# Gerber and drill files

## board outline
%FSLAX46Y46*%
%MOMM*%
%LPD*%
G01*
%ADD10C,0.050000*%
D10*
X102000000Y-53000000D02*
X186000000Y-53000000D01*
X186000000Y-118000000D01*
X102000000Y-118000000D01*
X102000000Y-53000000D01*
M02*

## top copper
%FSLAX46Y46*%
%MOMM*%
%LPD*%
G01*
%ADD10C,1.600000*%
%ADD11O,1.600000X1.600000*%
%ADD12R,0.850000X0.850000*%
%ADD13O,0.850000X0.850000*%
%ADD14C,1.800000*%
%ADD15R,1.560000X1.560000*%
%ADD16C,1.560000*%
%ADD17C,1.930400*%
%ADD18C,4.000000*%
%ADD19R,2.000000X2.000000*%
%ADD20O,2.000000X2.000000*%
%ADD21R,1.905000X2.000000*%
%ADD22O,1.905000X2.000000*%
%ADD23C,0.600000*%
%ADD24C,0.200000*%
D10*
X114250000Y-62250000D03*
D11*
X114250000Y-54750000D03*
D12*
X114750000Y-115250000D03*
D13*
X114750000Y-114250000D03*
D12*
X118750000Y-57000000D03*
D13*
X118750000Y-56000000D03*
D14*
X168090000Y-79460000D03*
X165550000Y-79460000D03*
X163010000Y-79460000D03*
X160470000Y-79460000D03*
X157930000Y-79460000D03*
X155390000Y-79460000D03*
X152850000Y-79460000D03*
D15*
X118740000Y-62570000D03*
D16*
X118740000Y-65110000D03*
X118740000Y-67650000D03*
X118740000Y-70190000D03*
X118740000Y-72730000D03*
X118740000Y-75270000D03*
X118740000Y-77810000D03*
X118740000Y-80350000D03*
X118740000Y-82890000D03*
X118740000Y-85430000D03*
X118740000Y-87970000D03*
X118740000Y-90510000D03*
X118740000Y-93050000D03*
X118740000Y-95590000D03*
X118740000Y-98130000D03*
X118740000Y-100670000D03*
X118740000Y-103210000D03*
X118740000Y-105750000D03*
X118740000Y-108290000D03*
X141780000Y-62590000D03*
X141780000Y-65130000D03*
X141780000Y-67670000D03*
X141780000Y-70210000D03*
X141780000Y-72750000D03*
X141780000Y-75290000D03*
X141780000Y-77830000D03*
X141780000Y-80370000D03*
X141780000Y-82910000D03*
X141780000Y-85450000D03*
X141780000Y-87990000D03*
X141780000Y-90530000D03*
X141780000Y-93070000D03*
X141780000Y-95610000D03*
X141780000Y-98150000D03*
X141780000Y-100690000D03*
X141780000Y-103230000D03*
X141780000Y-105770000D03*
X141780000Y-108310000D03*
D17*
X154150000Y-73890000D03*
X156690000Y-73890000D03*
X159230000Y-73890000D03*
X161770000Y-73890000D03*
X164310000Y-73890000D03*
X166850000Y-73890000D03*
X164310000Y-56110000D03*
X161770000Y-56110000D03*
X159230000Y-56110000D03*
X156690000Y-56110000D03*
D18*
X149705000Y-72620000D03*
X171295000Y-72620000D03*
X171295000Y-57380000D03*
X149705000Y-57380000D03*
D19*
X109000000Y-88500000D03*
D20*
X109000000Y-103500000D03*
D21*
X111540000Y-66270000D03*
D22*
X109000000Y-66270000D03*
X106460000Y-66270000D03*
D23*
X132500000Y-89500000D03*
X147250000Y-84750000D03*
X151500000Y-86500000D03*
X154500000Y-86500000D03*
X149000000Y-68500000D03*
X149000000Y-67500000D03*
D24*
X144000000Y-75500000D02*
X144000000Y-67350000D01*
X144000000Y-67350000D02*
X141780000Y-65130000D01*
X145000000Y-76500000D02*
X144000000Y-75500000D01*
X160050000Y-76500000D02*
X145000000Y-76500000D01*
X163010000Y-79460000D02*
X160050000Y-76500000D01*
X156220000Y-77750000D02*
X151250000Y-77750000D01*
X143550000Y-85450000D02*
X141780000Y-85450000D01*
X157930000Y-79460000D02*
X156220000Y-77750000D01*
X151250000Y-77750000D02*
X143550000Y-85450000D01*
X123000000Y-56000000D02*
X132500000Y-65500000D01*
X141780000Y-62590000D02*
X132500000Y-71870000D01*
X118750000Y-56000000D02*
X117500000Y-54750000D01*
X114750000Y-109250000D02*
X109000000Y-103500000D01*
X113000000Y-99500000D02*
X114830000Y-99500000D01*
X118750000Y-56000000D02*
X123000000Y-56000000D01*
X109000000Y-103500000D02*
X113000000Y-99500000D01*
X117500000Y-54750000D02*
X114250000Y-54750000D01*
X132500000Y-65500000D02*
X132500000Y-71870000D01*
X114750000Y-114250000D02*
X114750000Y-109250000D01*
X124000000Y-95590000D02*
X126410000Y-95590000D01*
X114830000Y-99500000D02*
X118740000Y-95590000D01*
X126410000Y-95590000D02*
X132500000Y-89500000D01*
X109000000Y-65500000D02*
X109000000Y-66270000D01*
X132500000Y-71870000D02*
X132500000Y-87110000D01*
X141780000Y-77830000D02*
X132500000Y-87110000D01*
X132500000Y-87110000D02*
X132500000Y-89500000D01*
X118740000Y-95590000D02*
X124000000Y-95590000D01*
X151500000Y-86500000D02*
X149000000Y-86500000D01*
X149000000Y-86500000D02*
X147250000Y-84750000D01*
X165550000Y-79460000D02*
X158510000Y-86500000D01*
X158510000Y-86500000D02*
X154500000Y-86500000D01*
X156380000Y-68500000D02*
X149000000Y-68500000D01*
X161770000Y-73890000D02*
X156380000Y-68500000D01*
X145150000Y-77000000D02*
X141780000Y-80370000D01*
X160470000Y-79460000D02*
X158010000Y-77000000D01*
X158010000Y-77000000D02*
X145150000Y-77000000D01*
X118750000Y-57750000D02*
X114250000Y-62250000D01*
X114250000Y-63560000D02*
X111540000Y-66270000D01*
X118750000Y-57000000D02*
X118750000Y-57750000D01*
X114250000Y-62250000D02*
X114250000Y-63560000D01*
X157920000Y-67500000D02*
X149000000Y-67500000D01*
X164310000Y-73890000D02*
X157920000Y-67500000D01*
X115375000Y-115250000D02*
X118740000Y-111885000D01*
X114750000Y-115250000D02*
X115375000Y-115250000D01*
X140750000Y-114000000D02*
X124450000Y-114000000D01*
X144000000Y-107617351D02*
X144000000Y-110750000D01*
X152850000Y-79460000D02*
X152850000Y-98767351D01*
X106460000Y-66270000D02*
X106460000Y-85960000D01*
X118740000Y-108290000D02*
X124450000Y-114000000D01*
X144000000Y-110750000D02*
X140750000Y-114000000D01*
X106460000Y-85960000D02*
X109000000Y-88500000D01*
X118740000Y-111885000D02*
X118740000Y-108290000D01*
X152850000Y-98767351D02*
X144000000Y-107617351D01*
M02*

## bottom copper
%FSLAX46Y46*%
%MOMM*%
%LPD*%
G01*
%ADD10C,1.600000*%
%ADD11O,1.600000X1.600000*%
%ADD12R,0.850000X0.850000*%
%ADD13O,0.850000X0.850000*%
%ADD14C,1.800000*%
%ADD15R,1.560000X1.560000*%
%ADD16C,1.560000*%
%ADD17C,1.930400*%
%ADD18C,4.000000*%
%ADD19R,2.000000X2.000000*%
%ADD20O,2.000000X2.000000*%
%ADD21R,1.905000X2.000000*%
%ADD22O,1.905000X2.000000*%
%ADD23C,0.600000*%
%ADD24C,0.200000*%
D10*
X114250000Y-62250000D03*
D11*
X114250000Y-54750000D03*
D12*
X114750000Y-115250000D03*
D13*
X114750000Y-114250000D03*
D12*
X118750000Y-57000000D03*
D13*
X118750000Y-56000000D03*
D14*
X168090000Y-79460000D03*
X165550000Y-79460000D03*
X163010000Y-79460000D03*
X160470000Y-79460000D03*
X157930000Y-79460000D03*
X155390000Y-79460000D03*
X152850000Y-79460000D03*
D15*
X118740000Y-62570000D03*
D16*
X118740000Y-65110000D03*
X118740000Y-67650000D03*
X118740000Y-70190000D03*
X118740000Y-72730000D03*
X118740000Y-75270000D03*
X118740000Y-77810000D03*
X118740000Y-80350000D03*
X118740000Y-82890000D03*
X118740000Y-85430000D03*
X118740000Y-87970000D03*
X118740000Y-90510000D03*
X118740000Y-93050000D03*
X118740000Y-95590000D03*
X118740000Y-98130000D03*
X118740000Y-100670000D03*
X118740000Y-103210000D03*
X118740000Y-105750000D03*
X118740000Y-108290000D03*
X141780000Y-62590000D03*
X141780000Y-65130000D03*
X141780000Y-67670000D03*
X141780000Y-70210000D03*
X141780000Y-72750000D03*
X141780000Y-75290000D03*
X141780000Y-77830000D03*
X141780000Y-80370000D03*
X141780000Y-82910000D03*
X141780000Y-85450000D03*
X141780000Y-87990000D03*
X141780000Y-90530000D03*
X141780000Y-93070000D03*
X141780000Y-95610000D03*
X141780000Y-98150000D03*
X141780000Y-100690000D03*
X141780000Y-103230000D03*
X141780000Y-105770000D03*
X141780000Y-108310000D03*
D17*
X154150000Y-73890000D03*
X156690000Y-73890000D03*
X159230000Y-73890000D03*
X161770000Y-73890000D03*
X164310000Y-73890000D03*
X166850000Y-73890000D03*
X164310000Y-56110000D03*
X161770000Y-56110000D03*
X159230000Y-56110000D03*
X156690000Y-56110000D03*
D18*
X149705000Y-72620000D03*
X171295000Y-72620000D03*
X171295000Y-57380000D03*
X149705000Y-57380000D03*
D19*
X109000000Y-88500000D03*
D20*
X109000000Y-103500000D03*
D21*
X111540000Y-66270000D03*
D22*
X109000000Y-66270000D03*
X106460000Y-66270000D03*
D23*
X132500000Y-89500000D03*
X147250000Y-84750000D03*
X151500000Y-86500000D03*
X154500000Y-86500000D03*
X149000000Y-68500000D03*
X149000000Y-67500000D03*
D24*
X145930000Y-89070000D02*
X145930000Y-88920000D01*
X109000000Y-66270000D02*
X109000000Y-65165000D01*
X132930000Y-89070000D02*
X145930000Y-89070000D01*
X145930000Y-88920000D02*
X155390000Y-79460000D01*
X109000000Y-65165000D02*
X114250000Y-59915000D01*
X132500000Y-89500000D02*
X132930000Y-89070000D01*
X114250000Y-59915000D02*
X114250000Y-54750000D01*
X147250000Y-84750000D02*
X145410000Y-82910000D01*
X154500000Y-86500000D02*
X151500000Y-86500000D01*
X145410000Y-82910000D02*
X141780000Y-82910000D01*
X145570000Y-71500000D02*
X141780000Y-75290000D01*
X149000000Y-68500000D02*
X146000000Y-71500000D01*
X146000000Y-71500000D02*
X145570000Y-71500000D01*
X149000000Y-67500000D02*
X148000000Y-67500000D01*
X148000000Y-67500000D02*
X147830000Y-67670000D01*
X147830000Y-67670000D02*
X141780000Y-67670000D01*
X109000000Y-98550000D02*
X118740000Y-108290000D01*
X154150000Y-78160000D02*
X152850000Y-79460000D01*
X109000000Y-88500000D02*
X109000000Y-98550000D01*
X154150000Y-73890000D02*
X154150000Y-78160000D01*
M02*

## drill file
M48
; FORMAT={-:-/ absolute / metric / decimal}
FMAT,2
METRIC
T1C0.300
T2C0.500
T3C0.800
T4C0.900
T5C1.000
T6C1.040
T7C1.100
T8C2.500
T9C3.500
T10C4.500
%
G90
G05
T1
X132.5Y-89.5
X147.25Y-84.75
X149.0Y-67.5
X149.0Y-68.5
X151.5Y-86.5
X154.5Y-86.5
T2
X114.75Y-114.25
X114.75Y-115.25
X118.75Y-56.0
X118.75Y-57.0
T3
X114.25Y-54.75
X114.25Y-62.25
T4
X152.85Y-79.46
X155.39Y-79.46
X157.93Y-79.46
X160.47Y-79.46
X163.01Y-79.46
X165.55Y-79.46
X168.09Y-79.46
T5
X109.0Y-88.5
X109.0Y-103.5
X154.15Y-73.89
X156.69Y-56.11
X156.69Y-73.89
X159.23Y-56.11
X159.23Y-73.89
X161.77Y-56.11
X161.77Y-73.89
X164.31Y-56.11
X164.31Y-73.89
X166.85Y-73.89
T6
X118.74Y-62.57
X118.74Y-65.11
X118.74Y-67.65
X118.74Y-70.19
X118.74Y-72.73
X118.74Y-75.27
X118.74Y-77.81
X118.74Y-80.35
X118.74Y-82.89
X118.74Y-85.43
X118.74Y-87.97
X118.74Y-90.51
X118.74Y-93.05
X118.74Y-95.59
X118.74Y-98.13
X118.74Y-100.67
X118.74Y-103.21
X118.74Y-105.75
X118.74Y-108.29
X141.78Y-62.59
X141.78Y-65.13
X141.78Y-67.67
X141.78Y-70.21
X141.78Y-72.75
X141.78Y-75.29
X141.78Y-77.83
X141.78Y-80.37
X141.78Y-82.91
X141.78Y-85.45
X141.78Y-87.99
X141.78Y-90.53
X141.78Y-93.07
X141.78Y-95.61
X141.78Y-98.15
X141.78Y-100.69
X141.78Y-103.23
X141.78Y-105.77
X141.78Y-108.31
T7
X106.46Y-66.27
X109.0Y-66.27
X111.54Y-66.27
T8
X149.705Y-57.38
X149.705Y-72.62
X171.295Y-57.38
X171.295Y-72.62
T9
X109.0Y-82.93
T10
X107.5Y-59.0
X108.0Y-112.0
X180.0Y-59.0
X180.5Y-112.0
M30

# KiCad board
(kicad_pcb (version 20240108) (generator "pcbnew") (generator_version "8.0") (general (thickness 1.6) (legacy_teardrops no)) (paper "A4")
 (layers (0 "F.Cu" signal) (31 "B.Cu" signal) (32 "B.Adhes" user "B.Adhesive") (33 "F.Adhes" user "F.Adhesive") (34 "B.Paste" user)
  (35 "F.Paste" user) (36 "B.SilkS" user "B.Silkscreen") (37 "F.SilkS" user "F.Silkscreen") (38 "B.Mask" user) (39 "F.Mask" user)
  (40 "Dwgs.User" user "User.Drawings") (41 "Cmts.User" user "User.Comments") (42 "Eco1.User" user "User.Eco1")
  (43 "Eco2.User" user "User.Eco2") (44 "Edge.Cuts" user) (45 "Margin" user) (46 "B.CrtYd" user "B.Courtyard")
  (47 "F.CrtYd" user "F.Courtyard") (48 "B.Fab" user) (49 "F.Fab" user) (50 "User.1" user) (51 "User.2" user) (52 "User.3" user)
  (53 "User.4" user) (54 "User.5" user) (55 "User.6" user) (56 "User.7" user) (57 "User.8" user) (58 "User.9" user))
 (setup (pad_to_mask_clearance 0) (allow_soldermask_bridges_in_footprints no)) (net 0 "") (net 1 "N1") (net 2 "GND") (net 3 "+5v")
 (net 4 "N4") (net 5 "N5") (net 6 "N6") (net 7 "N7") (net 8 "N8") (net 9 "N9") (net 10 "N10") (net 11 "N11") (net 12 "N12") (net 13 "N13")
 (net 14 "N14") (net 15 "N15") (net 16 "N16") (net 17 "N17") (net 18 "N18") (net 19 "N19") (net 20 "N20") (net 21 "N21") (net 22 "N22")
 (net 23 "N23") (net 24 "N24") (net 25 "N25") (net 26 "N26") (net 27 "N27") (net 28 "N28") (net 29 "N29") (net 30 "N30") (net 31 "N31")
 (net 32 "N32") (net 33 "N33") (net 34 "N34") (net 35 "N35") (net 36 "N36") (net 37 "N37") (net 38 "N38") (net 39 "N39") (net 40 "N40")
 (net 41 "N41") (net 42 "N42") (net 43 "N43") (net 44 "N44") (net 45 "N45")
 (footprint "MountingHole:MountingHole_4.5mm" (layer "F.Cu") (at 107.5 59)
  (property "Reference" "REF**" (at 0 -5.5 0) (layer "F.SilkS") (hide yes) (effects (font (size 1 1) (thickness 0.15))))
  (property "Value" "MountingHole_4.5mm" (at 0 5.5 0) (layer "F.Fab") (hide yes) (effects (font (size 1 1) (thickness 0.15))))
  (pad "" np_thru_hole circle (at 0 0) (size 4.5 4.5) (drill 4.5) (layers "*.Cu" "*.Mask")))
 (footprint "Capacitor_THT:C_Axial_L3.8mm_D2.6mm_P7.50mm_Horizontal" (layer "F.Cu") (at 114.25 62.25 90)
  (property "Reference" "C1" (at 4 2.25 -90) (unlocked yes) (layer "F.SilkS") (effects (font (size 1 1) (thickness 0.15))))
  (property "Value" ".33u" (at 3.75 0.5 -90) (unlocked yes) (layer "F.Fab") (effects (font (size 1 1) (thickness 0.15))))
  (pad "1" thru_hole circle (at 0 0 90) (size 1.6 1.6) (drill 0.8) (layers "*.Cu" "*.Mask") (remove_unused_layers no) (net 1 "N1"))
  (pad "2" thru_hole oval (at 7.5 0 90) (size 1.6 1.6) (drill 0.8) (layers "*.Cu" "*.Mask") (remove_unused_layers no) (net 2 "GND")))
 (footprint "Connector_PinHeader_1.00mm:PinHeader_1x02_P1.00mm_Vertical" (layer "F.Cu") (at 114.75 115.25 180)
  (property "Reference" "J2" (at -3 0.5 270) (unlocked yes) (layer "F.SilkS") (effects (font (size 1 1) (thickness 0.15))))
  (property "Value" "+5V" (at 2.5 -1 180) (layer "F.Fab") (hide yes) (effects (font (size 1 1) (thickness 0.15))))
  (pad "1" thru_hole rect (at 0 0 180) (size 0.85 0.85) (drill 0.5) (layers "*.Cu" "*.Mask") (remove_unused_layers no) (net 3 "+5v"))
  (pad "2" thru_hole oval (at 0 1 180) (size 0.85 0.85) (drill 0.5) (layers "*.Cu" "*.Mask") (remove_unused_layers no) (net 2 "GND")))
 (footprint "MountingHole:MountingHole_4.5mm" (layer "F.Cu") (at 180.5 112)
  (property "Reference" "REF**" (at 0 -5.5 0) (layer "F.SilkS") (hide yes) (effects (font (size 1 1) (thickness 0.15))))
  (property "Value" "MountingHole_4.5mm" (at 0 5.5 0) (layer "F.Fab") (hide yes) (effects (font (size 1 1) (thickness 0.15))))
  (pad "" np_thru_hole circle (at 0 0) (size 4.5 4.5) (drill 4.5) (layers "*.Cu" "*.Mask")))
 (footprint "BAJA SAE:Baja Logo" (layer "F.Cu") (at 181.25 79.5 -90)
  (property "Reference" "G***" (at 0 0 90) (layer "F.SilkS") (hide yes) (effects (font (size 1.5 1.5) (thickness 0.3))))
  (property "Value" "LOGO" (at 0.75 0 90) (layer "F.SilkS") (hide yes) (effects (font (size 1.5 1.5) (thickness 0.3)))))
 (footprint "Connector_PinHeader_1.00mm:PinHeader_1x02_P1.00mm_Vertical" (layer "F.Cu") (at 118.75 57 180)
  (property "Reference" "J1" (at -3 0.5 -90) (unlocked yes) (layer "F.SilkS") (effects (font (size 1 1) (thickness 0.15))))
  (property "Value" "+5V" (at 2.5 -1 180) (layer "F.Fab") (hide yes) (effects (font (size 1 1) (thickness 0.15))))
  (pad "1" thru_hole rect (at 0 0 180) (size 0.85 0.85) (drill 0.5) (layers "*.Cu" "*.Mask") (remove_unused_layers no) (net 1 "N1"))
  (pad "2" thru_hole oval (at 0 1 180) (size 0.85 0.85) (drill 0.5) (layers "*.Cu" "*.Mask") (remove_unused_layers no) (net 2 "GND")))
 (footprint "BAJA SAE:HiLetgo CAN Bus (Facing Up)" (layer "F.Cu") (at 160.5 97.5 -90)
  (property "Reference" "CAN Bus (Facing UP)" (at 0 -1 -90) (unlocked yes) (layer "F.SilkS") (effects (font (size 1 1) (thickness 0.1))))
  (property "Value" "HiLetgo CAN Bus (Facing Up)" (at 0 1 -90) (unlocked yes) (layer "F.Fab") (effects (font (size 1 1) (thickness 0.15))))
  (pad "1" thru_hole circle (at -18.04 -7.59 270) (size 1.8 1.8) (drill 0.9) (layers "*.Cu" "*.Mask") (remove_unused_layers no) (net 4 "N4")
   (solder_mask_margin 0.102))
  (pad "2" thru_hole circle (at -18.04 -5.05 270) (size 1.8 1.8) (drill 0.9) (layers "*.Cu" "*.Mask") (remove_unused_layers no) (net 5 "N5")
   (solder_mask_margin 0.102))
  (pad "3" thru_hole circle (at -18.04 -2.51 270) (size 1.8 1.8) (drill 0.9) (layers "*.Cu" "*.Mask") (remove_unused_layers no) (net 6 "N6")
   (solder_mask_margin 0.102))
  (pad "4" thru_hole circle (at -18.04 0.03 270) (size 1.8 1.8) (drill 0.9) (layers "*.Cu" "*.Mask") (remove_unused_layers no) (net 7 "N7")
   (solder_mask_margin 0.102))
  (pad "5" thru_hole circle (at -18.04 2.57 270) (size 1.8 1.8) (drill 0.9) (layers "*.Cu" "*.Mask") (remove_unused_layers no) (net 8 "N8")
   (solder_mask_margin 0.102))
  (pad "6" thru_hole circle (at -18.04 5.11 270) (size 1.8 1.8) (drill 0.9) (layers "*.Cu" "*.Mask") (remove_unused_layers no) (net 2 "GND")
   (solder_mask_margin 0.102))
  (pad "7" thru_hole circle (at -18.04 7.65 270) (size 1.8 1.8) (drill 0.9) (layers "*.Cu" "*.Mask") (remove_unused_layers no) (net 3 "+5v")
   (solder_mask_margin 0.102)))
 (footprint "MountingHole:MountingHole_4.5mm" (layer "F.Cu") (at 180 59)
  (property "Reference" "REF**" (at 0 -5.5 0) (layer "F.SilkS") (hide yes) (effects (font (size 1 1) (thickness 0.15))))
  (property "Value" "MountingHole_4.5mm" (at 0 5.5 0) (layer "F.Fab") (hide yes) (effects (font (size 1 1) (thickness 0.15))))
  (pad "" np_thru_hole circle (at 0 0) (size 4.5 4.5) (drill 4.5) (layers "*.Cu" "*.Mask")))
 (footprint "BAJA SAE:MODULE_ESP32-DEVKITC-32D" (layer "F.Cu") (at 130.5 81.5)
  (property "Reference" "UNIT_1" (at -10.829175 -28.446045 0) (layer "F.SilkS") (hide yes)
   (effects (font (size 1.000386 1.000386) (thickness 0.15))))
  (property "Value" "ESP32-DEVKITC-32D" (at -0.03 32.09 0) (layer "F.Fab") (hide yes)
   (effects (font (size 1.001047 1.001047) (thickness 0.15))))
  (pad "J2-1" thru_hole rect (at -11.76 -18.93) (size 1.56 1.56) (drill 1.04) (layers "*.Cu" "*.Mask") (remove_unused_layers no)
   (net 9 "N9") (solder_mask_margin 0.102))
  (pad "J2-2" thru_hole circle (at -11.76 -16.39) (size 1.56 1.56) (drill 1.04) (layers "*.Cu" "*.Mask") (remove_unused_layers no)
   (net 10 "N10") (solder_mask_margin 0.102))
  (pad "J2-3" thru_hole circle (at -11.76 -13.85) (size 1.56 1.56) (drill 1.04) (layers "*.Cu" "*.Mask") (remove_unused_layers no)
   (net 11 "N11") (solder_mask_margin 0.102))
  (pad "J2-4" thru_hole circle (at -11.76 -11.31) (size 1.56 1.56) (drill 1.04) (layers "*.Cu" "*.Mask") (remove_unused_layers no)
   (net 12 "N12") (solder_mask_margin 0.102))
  (pad "J2-5" thru_hole circle (at -11.76 -8.77) (size 1.56 1.56) (drill 1.04) (layers "*.Cu" "*.Mask") (remove_unused_layers no)
   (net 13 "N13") (solder_mask_margin 0.102))
  (pad "J2-6" thru_hole circle (at -11.76 -6.23) (size 1.56 1.56) (drill 1.04) (layers "*.Cu" "*.Mask") (remove_unused_layers no)
   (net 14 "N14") (solder_mask_margin 0.102))
  (pad "J2-7" thru_hole circle (at -11.76 -3.69) (size 1.56 1.56) (drill 1.04) (layers "*.Cu" "*.Mask") (remove_unused_layers no)
   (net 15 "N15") (solder_mask_margin 0.102))
  (pad "J2-8" thru_hole circle (at -11.76 -1.15) (size 1.56 1.56) (drill 1.04) (layers "*.Cu" "*.Mask") (remove_unused_layers no)
   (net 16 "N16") (solder_mask_margin 0.102))
  (pad "J2-9" thru_hole circle (at -11.76 1.39) (size 1.56 1.56) (drill 1.04) (layers "*.Cu" "*.Mask") (remove_unused_layers no)
   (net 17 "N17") (solder_mask_margin 0.102))
  (pad "J2-10" thru_hole circle (at -11.76 3.93) (size 1.56 1.56) (drill 1.04) (layers "*.Cu" "*.Mask") (remove_unused_layers no)
   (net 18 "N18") (solder_mask_margin 0.102))
  (pad "J2-11" thru_hole circle (at -11.76 6.47) (size 1.56 1.56) (drill 1.04) (layers "*.Cu" "*.Mask") (remove_unused_layers no)
   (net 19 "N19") (solder_mask_margin 0.102))
  (pad "J2-12" thru_hole circle (at -11.76 9.01) (size 1.56 1.56) (drill 1.04) (layers "*.Cu" "*.Mask") (remove_unused_layers no)
   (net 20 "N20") (solder_mask_margin 0.102))
  (pad "J2-13" thru_hole circle (at -11.76 11.55) (size 1.56 1.56) (drill 1.04) (layers "*.Cu" "*.Mask") (remove_unused_layers no)
   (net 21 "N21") (solder_mask_margin 0.102))
  (pad "J2-14" thru_hole circle (at -11.76 14.09) (size 1.56 1.56) (drill 1.04) (layers "*.Cu" "*.Mask") (remove_unused_layers no)
   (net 2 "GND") (solder_mask_margin 0.102))
  (pad "J2-15" thru_hole circle (at -11.76 16.63) (size 1.56 1.56) (drill 1.04) (layers "*.Cu" "*.Mask") (remove_unused_layers no)
   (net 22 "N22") (solder_mask_margin 0.102))
  (pad "J2-16" thru_hole circle (at -11.76 19.17) (size 1.56 1.56) (drill 1.04) (layers "*.Cu" "*.Mask") (remove_unused_layers no)
   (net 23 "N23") (solder_mask_margin 0.102))
  (pad "J2-17" thru_hole circle (at -11.76 21.71) (size 1.56 1.56) (drill 1.04) (layers "*.Cu" "*.Mask") (remove_unused_layers no)
   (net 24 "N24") (solder_mask_margin 0.102))
  (pad "J2-18" thru_hole circle (at -11.76 24.25) (size 1.56 1.56) (drill 1.04) (layers "*.Cu" "*.Mask") (remove_unused_layers no)
   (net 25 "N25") (solder_mask_margin 0.102))
  (pad "J2-19" thru_hole circle (at -11.76 26.79) (size 1.56 1.56) (drill 1.04) (layers "*.Cu" "*.Mask") (remove_unused_layers no)
   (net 3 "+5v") (solder_mask_margin 0.102))
  (pad "J3-1" thru_hole circle (at 11.28 -18.91) (size 1.56 1.56) (drill 1.04) (layers "*.Cu" "*.Mask") (remove_unused_layers no)
   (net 2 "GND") (solder_mask_margin 0.102))
  (pad "J3-2" thru_hole circle (at 11.28 -16.37) (size 1.56 1.56) (drill 1.04) (layers "*.Cu" "*.Mask") (remove_unused_layers no)
   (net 6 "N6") (solder_mask_margin 0.102))
  (pad "J3-3" thru_hole circle (at 11.28 -13.83) (size 1.56 1.56) (drill 1.04) (layers "*.Cu" "*.Mask") (remove_unused_layers no)
   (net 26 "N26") (solder_mask_margin 0.102))
  (pad "J3-4" thru_hole circle (at 11.28 -11.29) (size 1.56 1.56) (drill 1.04) (layers "*.Cu" "*.Mask") (remove_unused_layers no)
   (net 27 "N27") (solder_mask_margin 0.102))
  (pad "J3-5" thru_hole circle (at 11.28 -8.75) (size 1.56 1.56) (drill 1.04) (layers "*.Cu" "*.Mask") (remove_unused_layers no)
   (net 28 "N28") (solder_mask_margin 0.102))
  (pad "J3-6" thru_hole circle (at 11.28 -6.21) (size 1.56 1.56) (drill 1.04) (layers "*.Cu" "*.Mask") (remove_unused_layers no)
   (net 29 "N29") (solder_mask_margin 0.102))
  (pad "J3-7" thru_hole circle (at 11.28 -3.67) (size 1.56 1.56) (drill 1.04) (layers "*.Cu" "*.Mask") (remove_unused_layers no)
   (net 2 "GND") (solder_mask_margin 0.102))
  (pad "J3-8" thru_hole circle (at 11.28 -1.13) (size 1.56 1.56) (drill 1.04) (layers "*.Cu" "*.Mask") (remove_unused_layers no)
   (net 7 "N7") (solder_mask_margin 0.102))
  (pad "J3-9" thru_hole circle (at 11.28 1.41) (size 1.56 1.56) (drill 1.04) (layers "*.Cu" "*.Mask") (remove_unused_layers no) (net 5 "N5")
   (solder_mask_margin 0.102))
  (pad "J3-10" thru_hole circle (at 11.28 3.95) (size 1.56 1.56) (drill 1.04) (layers "*.Cu" "*.Mask") (remove_unused_layers no)
   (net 8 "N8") (solder_mask_margin 0.102))
  (pad "J3-11" thru_hole circle (at 11.28 6.49) (size 1.56 1.56) (drill 1.04) (layers "*.Cu" "*.Mask") (remove_unused_layers no)
   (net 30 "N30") (solder_mask_margin 0.102))
  (pad "J3-12" thru_hole circle (at 11.28 9.03) (size 1.56 1.56) (drill 1.04) (layers "*.Cu" "*.Mask") (remove_unused_layers no)
   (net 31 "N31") (solder_mask_margin 0.102))
  (pad "J3-13" thru_hole circle (at 11.28 11.57) (size 1.56 1.56) (drill 1.04) (layers "*.Cu" "*.Mask") (remove_unused_layers no)
   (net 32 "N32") (solder_mask_margin 0.102))
  (pad "J3-14" thru_hole circle (at 11.28 14.11) (size 1.56 1.56) (drill 1.04) (layers "*.Cu" "*.Mask") (remove_unused_layers no)
   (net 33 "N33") (solder_mask_margin 0.102))
  (pad "J3-15" thru_hole circle (at 11.28 16.65) (size 1.56 1.56) (drill 1.04) (layers "*.Cu" "*.Mask") (remove_unused_layers no)
   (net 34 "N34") (solder_mask_margin 0.102))
  (pad "J3-16" thru_hole circle (at 11.28 19.19) (size 1.56 1.56) (drill 1.04) (layers "*.Cu" "*.Mask") (remove_unused_layers no)
   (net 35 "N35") (solder_mask_margin 0.102))
  (pad "J3-17" thru_hole circle (at 11.28 21.73) (size 1.56 1.56) (drill 1.04) (layers "*.Cu" "*.Mask") (remove_unused_layers no)
   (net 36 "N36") (solder_mask_margin 0.102))
  (pad "J3-18" thru_hole circle (at 11.28 24.27) (size 1.56 1.56) (drill 1.04) (layers "*.Cu" "*.Mask") (remove_unused_layers no)
   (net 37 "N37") (solder_mask_margin 0.102))
  (pad "J3-19" thru_hole circle (at 11.28 26.81) (size 1.56 1.56) (drill 1.04) (layers "*.Cu" "*.Mask") (remove_unused_layers no)
   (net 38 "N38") (solder_mask_margin 0.102)))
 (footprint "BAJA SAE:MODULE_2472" (layer "F.Cu") (at 160.5 65)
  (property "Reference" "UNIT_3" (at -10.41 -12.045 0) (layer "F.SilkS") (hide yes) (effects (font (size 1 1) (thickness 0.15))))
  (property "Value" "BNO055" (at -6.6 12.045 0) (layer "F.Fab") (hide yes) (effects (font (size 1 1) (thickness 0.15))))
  (pad "1" thru_hole circle (at -6.35 8.89) (size 1.9304 1.9304) (drill 1) (layers "*.Cu" "*.Mask") (remove_unused_layers no) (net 3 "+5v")
   (solder_mask_margin 0.102))
  (pad "2" thru_hole circle (at -3.81 8.89) (size 1.9304 1.9304) (drill 1) (layers "*.Cu" "*.Mask") (remove_unused_layers no) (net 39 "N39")
   (solder_mask_margin 0.102))
  (pad "3" thru_hole circle (at -1.27 8.89) (size 1.9304 1.9304) (drill 1) (layers "*.Cu" "*.Mask") (remove_unused_layers no) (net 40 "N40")
   (solder_mask_margin 0.102))
  (pad "4" thru_hole circle (at 1.27 8.89) (size 1.9304 1.9304) (drill 1) (layers "*.Cu" "*.Mask") (remove_unused_layers no) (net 29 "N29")
   (solder_mask_margin 0.102))
  (pad "5" thru_hole circle (at 3.81 8.89) (size 1.9304 1.9304) (drill 1) (layers "*.Cu" "*.Mask") (remove_unused_layers no) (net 26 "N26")
   (solder_mask_margin 0.102))
  (pad "6" thru_hole circle (at 6.35 8.89) (size 1.9304 1.9304) (drill 1) (layers "*.Cu" "*.Mask") (remove_unused_layers no) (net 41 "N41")
   (solder_mask_margin 0.102))
  (pad "7" thru_hole circle (at 3.81 -8.89) (size 1.9304 1.9304) (drill 1) (layers "*.Cu" "*.Mask") (remove_unused_layers no) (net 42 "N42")
   (solder_mask_margin 0.102))
  (pad "8" thru_hole circle (at 1.27 -8.89) (size 1.9304 1.9304) (drill 1) (layers "*.Cu" "*.Mask") (remove_unused_layers no) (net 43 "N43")
   (solder_mask_margin 0.102))
  (pad "9" thru_hole circle (at -1.27 -8.89) (size 1.9304 1.9304) (drill 1) (layers "*.Cu" "*.Mask") (remove_unused_layers no)
   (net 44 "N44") (solder_mask_margin 0.102))
  (pad "10" thru_hole circle (at -3.81 -8.89) (size 1.9304 1.9304) (drill 1) (layers "*.Cu" "*.Mask") (remove_unused_layers no)
   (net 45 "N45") (solder_mask_margin 0.102))
  (pad "SH1" thru_hole circle (at -10.795 7.62) (size 4 4) (drill 2.5) (layers "*.Cu" "*.Mask") (remove_unused_layers no)
   (solder_mask_margin 0.102))
  (pad "SH2" thru_hole circle (at 10.795 7.62) (size 4 4) (drill 2.5) (layers "*.Cu" "*.Mask") (remove_unused_layers no)
   (solder_mask_margin 0.102))
  (pad "SH3" thru_hole circle (at 10.795 -7.62) (size 4 4) (drill 2.5) (layers "*.Cu" "*.Mask") (remove_unused_layers no)
   (solder_mask_margin 0.102))
  (pad "SH4" thru_hole circle (at -10.795 -7.62) (size 4 4) (drill 2.5) (layers "*.Cu" "*.Mask") (remove_unused_layers no)
   (solder_mask_margin 0.102)))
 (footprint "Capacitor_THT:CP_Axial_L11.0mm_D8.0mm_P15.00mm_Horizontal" (layer "F.Cu") (at 109 88.5 -90)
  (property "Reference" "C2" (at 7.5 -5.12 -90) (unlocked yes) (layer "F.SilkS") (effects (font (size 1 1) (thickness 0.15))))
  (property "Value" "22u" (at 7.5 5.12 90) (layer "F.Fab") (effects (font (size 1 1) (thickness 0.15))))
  (pad "1" thru_hole rect (at 0 0 270) (size 2 2) (drill 1) (layers "*.Cu" "*.Mask") (remove_unused_layers no) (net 3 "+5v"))
  (pad "2" thru_hole oval (at 15 0 270) (size 2 2) (drill 1) (layers "*.Cu" "*.Mask") (remove_unused_layers no) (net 2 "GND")))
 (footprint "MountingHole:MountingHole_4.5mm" (layer "F.Cu") (at 108 112)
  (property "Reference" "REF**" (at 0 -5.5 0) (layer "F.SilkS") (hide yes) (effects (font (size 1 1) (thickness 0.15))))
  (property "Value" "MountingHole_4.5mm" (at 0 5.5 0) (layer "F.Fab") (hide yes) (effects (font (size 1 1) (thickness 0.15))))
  (pad "" np_thru_hole circle (at 0 0) (size 4.5 4.5) (drill 4.5) (layers "*.Cu" "*.Mask")))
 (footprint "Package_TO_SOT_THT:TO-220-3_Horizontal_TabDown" (layer "F.Cu") (at 111.54 66.27 180)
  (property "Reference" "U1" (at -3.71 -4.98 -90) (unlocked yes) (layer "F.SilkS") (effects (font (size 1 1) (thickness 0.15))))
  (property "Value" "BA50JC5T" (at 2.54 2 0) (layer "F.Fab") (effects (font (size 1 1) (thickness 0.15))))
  (pad "" np_thru_hole oval (at 2.54 -16.66 180) (size 3.5 3.5) (drill 3.5) (layers "*.Cu" "*.Mask"))
  (pad "1" thru_hole rect (at 0 0 180) (size 1.905 2) (drill 1.1) (layers "*.Cu" "*.Mask") (remove_unused_layers no) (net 1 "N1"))
  (pad "2" thru_hole oval (at 2.54 0 180) (size 1.905 2) (drill 1.1) (layers "*.Cu" "*.Mask") (remove_unused_layers no) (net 2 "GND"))
  (pad "3" thru_hole oval (at 5.08 0 180) (size 1.905 2) (drill 1.1) (layers "*.Cu" "*.Mask") (remove_unused_layers no) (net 3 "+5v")))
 (gr_rect (start 102 53) (end 186 118) (stroke (width 0.05) (type default)) (fill none) (layer "Edge.Cuts"))
 (segment (start 144 75.5) (end 144 67.35) (width 0.2) (layer "F.Cu") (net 6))
 (segment (start 144 67.35) (end 141.78 65.13) (width 0.2) (layer "F.Cu") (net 6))
 (segment (start 145 76.5) (end 144 75.5) (width 0.2) (layer "F.Cu") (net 6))
 (segment (start 160.05 76.5) (end 145 76.5) (width 0.2) (layer "F.Cu") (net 6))
 (segment (start 163.01 79.46) (end 160.05 76.5) (width 0.2) (layer "F.Cu") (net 6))
 (segment (start 156.22 77.75) (end 151.25 77.75) (width 0.2) (layer "F.Cu") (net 8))
 (segment (start 143.55 85.45) (end 141.78 85.45) (width 0.2) (layer "F.Cu") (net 8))
 (segment (start 157.93 79.46) (end 156.22 77.75) (width 0.2) (layer "F.Cu") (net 8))
 (segment (start 151.25 77.75) (end 143.55 85.45) (width 0.2) (layer "F.Cu") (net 8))
 (segment (start 123 56) (end 132.5 65.5) (width 0.2) (layer "F.Cu") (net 2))
 (segment (start 141.78 62.59) (end 132.5 71.87) (width 0.2) (layer "F.Cu") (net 2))
 (segment (start 118.75 56) (end 117.5 54.75) (width 0.2) (layer "F.Cu") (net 2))
 (segment (start 114.75 109.25) (end 109 103.5) (width 0.2) (layer "F.Cu") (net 2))
 (segment (start 113 99.5) (end 114.83 99.5) (width 0.2) (layer "F.Cu") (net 2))
 (segment (start 118.75 56) (end 123 56) (width 0.2) (layer "F.Cu") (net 2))
 (segment (start 109 103.5) (end 113 99.5) (width 0.2) (layer "F.Cu") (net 2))
 (segment (start 117.5 54.75) (end 114.25 54.75) (width 0.2) (layer "F.Cu") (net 2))
 (segment (start 132.5 65.5) (end 132.5 71.87) (width 0.2) (layer "F.Cu") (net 2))
 (segment (start 114.75 114.25) (end 114.75 109.25) (width 0.2) (layer "F.Cu") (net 2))
 (segment (start 124 95.59) (end 126.41 95.59) (width 0.2) (layer "F.Cu") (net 2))
 (segment (start 114.83 99.5) (end 118.74 95.59) (width 0.2) (layer "F.Cu") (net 2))
 (segment (start 126.41 95.59) (end 132.5 89.5) (width 0.2) (layer "F.Cu") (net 2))
 (segment (start 109 65.5) (end 109 66.27) (width 0.2) (layer "F.Cu") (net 2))
 (segment (start 132.5 71.87) (end 132.5 87.11) (width 0.2) (layer "F.Cu") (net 2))
 (segment (start 141.78 77.83) (end 132.5 87.11) (width 0.2) (layer "F.Cu") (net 2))
 (segment (start 132.5 87.11) (end 132.5 89.5) (width 0.2) (layer "F.Cu") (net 2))
 (segment (start 118.74 95.59) (end 124 95.59) (width 0.2) (layer "F.Cu") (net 2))
 (via (at 132.5 89.5) (size 0.6) (drill 0.3) (layers "F.Cu" "B.Cu") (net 2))
 (segment (start 145.93 89.07) (end 145.93 88.92) (width 0.2) (layer "B.Cu") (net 2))
 (segment (start 109 66.27) (end 109 65.165) (width 0.2) (layer "B.Cu") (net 2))
 (segment (start 132.93 89.07) (end 145.93 89.07) (width 0.2) (layer "B.Cu") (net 2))
 (segment (start 145.93 88.92) (end 155.39 79.46) (width 0.2) (layer "B.Cu") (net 2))
 (segment (start 109 65.165) (end 114.25 59.915) (width 0.2) (layer "B.Cu") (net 2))
 (segment (start 132.5 89.5) (end 132.93 89.07) (width 0.2) (layer "B.Cu") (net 2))
 (segment (start 114.25 59.915) (end 114.25 54.75) (width 0.2) (layer "B.Cu") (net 2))
 (segment (start 151.5 86.5) (end 149 86.5) (width 0.2) (layer "F.Cu") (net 5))
 (segment (start 149 86.5) (end 147.25 84.75) (width 0.2) (layer "F.Cu") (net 5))
 (segment (start 165.55 79.46) (end 158.51 86.5) (width 0.2) (layer "F.Cu") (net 5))
 (segment (start 158.51 86.5) (end 154.5 86.5) (width 0.2) (layer "F.Cu") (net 5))
 (via (at 147.25 84.75) (size 0.6) (drill 0.3) (layers "F.Cu" "B.Cu") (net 5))
 (via (at 151.5 86.5) (size 0.6) (drill 0.3) (layers "F.Cu" "B.Cu") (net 5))
 (via (at 154.5 86.5) (size 0.6) (drill 0.3) (layers "F.Cu" "B.Cu") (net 5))
 (segment (start 147.25 84.75) (end 145.41 82.91) (width 0.2) (layer "B.Cu") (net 5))
 (segment (start 154.5 86.5) (end 151.5 86.5) (width 0.2) (layer "B.Cu") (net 5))
 (segment (start 145.41 82.91) (end 141.78 82.91) (width 0.2) (layer "B.Cu") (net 5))
 (segment (start 156.38 68.5) (end 149 68.5) (width 0.2) (layer "F.Cu") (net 29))
 (segment (start 161.77 73.89) (end 156.38 68.5) (width 0.2) (layer "F.Cu") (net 29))
 (via (at 149 68.5) (size 0.6) (drill 0.3) (layers "F.Cu" "B.Cu") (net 29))
 (segment (start 145.57 71.5) (end 141.78 75.29) (width 0.2) (layer "B.Cu") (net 29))
 (segment (start 149 68.5) (end 146 71.5) (width 0.2) (layer "B.Cu") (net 29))
 (segment (start 146 71.5) (end 145.57 71.5) (width 0.2) (layer "B.Cu") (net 29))
 (segment (start 145.15 77) (end 141.78 80.37) (width 0.2) (layer "F.Cu") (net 7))
 (segment (start 160.47 79.46) (end 158.01 77) (width 0.2) (layer "F.Cu") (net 7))
 (segment (start 158.01 77) (end 145.15 77) (width 0.2) (layer "F.Cu") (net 7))
 (segment (start 118.75 57.75) (end 114.25 62.25) (width 0.2) (layer "F.Cu") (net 1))
 (segment (start 114.25 63.56) (end 111.54 66.27) (width 0.2) (layer "F.Cu") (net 1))
 (segment (start 118.75 57) (end 118.75 57.75) (width 0.2) (layer "F.Cu") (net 1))
 (segment (start 114.25 62.25) (end 114.25 63.56) (width 0.2) (layer "F.Cu") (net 1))
 (segment (start 157.92 67.5) (end 149 67.5) (width 0.2) (layer "F.Cu") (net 26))
 (segment (start 164.31 73.89) (end 157.92 67.5) (width 0.2) (layer "F.Cu") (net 26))
 (via (at 149 67.5) (size 0.6) (drill 0.3) (layers "F.Cu" "B.Cu") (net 26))
 (segment (start 149 67.5) (end 148 67.5) (width 0.2) (layer "B.Cu") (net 26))
 (segment (start 148 67.5) (end 147.83 67.67) (width 0.2) (layer "B.Cu") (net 26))
 (segment (start 147.83 67.67) (end 141.78 67.67) (width 0.2) (layer "B.Cu") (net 26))
 (segment (start 115.375 115.25) (end 118.74 111.885) (width 0.2) (layer "F.Cu") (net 3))
 (segment (start 114.75 115.25) (end 115.375 115.25) (width 0.2) (layer "F.Cu") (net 3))
 (segment (start 140.75 114) (end 124.45 114) (width 0.2) (layer "F.Cu") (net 3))
 (segment (start 144 107.617351) (end 144 110.75) (width 0.2) (layer "F.Cu") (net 3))
 (segment (start 152.85 79.46) (end 152.85 98.767351) (width 0.2) (layer "F.Cu") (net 3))
 (segment (start 106.46 66.27) (end 106.46 85.96) (width 0.2) (layer "F.Cu") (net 3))
 (segment (start 118.74 108.29) (end 124.45 114) (width 0.2) (layer "F.Cu") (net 3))
 (segment (start 144 110.75) (end 140.75 114) (width 0.2) (layer "F.Cu") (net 3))
 (segment (start 106.46 85.96) (end 109 88.5) (width 0.2) (layer "F.Cu") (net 3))
 (segment (start 118.74 111.885) (end 118.74 108.29) (width 0.2) (layer "F.Cu") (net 3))
 (segment (start 152.85 98.767351) (end 144 107.617351) (width 0.2) (layer "F.Cu") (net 3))
 (segment (start 109 98.55) (end 118.74 108.29) (width 0.2) (layer "B.Cu") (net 3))
 (segment (start 154.15 78.16) (end 152.85 79.46) (width 0.2) (layer "B.Cu") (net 3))
 (segment (start 109 88.5) (end 109 98.55) (width 0.2) (layer "B.Cu") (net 3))
 (segment (start 154.15 73.89) (end 154.15 78.16) (width 0.2) (layer "B.Cu") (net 3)))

